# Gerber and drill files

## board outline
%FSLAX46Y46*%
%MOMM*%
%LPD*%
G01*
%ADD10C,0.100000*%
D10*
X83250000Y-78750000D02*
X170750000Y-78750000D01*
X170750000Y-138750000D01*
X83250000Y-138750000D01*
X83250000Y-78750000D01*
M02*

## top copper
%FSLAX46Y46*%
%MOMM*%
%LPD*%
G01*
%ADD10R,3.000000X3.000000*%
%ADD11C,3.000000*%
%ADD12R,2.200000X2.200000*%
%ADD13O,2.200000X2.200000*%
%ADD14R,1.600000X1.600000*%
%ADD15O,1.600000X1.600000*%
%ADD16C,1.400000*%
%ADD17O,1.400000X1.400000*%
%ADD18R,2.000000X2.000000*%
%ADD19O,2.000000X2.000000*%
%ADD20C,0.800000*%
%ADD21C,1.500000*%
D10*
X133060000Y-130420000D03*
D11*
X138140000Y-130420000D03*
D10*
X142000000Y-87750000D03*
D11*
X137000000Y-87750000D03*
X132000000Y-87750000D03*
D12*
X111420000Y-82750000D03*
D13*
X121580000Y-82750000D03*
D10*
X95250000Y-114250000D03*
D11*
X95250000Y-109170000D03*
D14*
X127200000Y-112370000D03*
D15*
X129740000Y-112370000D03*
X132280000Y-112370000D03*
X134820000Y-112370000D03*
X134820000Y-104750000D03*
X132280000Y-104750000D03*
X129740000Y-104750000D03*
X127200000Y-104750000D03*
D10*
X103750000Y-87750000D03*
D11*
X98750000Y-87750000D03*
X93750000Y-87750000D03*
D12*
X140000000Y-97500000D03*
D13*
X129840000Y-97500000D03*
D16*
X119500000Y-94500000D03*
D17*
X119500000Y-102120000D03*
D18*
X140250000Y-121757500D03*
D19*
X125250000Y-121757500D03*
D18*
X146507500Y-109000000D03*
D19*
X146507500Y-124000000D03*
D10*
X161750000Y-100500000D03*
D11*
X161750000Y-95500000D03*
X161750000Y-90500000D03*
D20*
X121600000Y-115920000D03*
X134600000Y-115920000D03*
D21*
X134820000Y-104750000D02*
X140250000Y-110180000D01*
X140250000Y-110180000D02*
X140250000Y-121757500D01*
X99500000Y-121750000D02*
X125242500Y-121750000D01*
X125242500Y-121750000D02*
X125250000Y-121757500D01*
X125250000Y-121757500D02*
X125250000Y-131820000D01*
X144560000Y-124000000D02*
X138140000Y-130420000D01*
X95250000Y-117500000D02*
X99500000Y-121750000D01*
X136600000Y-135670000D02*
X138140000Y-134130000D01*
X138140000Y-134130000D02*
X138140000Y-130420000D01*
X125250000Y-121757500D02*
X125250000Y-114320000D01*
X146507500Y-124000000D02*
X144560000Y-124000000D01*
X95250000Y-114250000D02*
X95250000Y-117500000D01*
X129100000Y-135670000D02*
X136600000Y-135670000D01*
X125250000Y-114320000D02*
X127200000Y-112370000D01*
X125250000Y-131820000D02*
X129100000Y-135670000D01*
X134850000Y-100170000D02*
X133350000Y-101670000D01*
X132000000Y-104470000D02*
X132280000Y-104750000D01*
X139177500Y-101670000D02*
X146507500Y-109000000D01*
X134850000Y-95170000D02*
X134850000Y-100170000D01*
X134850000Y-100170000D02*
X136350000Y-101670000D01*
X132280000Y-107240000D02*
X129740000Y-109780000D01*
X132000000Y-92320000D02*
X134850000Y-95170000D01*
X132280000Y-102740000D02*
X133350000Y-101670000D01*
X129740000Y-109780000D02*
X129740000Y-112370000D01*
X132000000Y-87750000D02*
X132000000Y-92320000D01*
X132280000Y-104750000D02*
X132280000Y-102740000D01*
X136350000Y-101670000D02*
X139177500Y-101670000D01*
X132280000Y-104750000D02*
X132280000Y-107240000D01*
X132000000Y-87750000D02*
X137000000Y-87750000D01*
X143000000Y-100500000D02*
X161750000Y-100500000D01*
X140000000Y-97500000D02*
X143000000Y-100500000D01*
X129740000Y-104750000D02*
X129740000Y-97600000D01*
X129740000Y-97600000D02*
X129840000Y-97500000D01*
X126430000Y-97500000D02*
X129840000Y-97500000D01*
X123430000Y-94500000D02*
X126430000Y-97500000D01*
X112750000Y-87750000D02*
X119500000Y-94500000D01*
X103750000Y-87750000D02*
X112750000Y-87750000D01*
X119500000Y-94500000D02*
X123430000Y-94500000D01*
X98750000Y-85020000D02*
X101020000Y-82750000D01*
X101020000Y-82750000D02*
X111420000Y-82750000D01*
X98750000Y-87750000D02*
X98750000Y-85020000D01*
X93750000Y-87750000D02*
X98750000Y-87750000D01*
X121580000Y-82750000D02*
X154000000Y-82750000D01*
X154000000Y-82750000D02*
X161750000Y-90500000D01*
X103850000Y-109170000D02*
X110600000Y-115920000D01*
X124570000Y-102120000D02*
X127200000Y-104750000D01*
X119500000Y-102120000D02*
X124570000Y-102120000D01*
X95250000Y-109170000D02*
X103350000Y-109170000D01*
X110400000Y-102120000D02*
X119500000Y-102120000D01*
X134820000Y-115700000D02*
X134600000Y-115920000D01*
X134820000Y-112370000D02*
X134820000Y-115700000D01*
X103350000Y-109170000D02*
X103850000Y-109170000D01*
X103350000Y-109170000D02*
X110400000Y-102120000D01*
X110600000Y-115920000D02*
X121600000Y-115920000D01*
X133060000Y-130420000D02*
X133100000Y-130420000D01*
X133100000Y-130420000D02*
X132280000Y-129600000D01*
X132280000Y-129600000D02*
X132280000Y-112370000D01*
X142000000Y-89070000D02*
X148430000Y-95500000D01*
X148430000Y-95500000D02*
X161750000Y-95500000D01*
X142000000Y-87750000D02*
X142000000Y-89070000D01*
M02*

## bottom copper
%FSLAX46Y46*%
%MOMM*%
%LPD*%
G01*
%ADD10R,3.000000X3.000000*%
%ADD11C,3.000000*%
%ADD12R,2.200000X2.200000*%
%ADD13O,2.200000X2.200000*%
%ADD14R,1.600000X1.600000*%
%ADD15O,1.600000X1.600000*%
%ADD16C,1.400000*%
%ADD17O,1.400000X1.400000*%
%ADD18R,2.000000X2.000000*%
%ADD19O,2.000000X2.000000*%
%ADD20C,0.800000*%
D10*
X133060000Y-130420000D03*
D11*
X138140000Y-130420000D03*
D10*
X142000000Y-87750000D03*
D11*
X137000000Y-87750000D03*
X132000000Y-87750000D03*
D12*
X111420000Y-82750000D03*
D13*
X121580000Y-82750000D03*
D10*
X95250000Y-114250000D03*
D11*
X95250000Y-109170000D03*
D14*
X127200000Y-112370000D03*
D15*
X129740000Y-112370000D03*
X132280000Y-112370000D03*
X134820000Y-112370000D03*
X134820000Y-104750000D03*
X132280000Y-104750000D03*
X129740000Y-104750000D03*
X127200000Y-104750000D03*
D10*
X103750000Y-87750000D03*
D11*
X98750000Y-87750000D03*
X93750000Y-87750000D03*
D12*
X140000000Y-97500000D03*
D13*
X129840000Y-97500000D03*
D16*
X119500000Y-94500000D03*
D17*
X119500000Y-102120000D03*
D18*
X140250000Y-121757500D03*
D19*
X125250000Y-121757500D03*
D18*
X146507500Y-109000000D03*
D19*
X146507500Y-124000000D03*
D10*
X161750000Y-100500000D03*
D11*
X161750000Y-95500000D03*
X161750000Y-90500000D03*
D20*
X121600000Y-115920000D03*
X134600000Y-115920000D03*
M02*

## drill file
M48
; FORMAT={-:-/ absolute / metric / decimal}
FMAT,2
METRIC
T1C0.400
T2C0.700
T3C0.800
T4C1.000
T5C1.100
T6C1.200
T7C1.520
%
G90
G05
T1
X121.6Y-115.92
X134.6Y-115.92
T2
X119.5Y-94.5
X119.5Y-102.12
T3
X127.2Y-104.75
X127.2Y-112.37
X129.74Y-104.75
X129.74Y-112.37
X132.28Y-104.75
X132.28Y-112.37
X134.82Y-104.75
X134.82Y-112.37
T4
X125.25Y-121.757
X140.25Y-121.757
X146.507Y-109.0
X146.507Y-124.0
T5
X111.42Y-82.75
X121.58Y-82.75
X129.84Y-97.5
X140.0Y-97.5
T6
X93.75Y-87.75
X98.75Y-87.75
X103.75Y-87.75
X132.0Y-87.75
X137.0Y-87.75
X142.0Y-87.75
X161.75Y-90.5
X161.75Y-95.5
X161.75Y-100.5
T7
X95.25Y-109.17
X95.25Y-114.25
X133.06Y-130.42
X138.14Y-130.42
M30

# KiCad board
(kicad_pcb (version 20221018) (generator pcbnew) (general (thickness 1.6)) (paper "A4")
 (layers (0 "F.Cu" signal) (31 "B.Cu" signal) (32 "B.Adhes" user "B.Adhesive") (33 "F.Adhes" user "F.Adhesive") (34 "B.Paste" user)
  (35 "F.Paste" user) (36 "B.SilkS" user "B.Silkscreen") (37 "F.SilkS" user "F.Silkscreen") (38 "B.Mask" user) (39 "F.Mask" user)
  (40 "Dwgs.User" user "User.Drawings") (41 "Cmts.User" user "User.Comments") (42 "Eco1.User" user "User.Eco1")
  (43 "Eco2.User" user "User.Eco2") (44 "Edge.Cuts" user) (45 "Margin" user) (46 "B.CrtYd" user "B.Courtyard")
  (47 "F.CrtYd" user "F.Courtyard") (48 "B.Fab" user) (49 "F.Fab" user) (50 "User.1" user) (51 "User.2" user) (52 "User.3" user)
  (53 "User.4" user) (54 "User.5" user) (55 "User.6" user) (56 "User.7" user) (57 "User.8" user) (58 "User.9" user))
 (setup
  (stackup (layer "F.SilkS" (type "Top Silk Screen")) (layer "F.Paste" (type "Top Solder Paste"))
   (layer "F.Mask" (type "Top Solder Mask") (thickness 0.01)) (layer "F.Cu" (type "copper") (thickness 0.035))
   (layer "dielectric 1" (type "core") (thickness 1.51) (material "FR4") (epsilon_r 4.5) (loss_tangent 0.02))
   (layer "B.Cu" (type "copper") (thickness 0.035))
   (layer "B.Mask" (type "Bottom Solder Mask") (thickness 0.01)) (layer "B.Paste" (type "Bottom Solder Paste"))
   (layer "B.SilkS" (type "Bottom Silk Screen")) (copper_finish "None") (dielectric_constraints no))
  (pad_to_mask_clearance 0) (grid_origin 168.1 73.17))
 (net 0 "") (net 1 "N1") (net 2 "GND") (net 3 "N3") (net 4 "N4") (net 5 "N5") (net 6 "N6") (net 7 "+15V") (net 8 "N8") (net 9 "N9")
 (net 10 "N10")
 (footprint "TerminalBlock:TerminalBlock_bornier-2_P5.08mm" (layer "F.Cu") (at 133.06 130.42)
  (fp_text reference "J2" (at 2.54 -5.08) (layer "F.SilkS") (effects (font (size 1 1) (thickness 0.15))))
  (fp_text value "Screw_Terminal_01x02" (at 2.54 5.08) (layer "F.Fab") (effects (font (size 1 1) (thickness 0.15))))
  (pad "1" thru_hole rect (at 0 0) (size 3 3) (drill 1.52) (layers "*.Cu" "*.Mask") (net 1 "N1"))
  (pad "2" thru_hole circle (at 5.08 0) (size 3 3) (drill 1.52) (layers "*.Cu" "*.Mask") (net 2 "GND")))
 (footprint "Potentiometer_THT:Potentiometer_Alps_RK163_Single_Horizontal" (layer "F.Cu") (at 142 87.75 -90)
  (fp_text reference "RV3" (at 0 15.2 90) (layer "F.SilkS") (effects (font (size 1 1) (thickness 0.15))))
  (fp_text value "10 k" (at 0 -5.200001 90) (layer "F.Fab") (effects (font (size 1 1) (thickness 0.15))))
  (pad "1" thru_hole rect (at 0 0 90) (size 3 3) (drill 1.2) (layers "*.Cu" "*.Mask") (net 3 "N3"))
  (pad "2" thru_hole circle (at 0 5 90) (size 3 3) (drill 1.2) (layers "*.Cu" "*.Mask") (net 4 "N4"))
  (pad "3" thru_hole circle (at 0 10 90) (size 3 3) (drill 1.2) (layers "*.Cu" "*.Mask") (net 4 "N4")))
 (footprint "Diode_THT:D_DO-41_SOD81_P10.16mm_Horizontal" (layer "F.Cu") (at 111.42 82.75)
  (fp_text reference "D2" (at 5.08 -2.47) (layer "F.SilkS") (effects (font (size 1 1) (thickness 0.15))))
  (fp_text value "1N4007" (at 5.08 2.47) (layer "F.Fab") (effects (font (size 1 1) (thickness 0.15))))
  (pad "1" thru_hole rect (at 0 0) (size 2.2 2.2) (drill 1.1) (layers "*.Cu" "*.Mask") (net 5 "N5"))
  (pad "2" thru_hole oval (at 10.16 0) (size 2.2 2.2) (drill 1.1) (layers "*.Cu" "*.Mask") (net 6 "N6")))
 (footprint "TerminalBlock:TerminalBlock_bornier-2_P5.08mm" (layer "F.Cu") (at 95.25 114.25 90)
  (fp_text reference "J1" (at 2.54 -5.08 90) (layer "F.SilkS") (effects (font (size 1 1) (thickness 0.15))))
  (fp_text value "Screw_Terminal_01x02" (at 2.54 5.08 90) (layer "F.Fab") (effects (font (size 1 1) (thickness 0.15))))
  (pad "1" thru_hole rect (at 0 0 90) (size 3 3) (drill 1.52) (layers "*.Cu" "*.Mask") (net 2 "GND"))
  (pad "2" thru_hole circle (at 5.08 0 90) (size 3 3) (drill 1.52) (layers "*.Cu" "*.Mask") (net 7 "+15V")))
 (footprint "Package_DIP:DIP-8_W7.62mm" (layer "F.Cu") (at 127.2 112.37 90)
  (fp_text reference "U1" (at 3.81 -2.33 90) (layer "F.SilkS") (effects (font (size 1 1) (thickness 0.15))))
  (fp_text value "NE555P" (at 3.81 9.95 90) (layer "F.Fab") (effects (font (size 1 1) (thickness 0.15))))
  (pad "1" thru_hole rect (at 0 0 90) (size 1.6 1.6) (drill 0.8) (layers "*.Cu" "*.Mask") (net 2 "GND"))
  (pad "2" thru_hole oval (at 0 2.54 90) (size 1.6 1.6) (drill 0.8) (layers "*.Cu" "*.Mask") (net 4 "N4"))
  (pad "3" thru_hole oval (at 0 5.08 90) (size 1.6 1.6) (drill 0.8) (layers "*.Cu" "*.Mask") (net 1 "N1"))
  (pad "4" thru_hole oval (at 0 7.62 90) (size 1.6 1.6) (drill 0.8) (layers "*.Cu" "*.Mask") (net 7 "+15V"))
  (pad "5" thru_hole oval (at 7.62 7.62 90) (size 1.6 1.6) (drill 0.8) (layers "*.Cu" "*.Mask") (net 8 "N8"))
  (pad "6" thru_hole oval (at 7.62 5.08 90) (size 1.6 1.6) (drill 0.8) (layers "*.Cu" "*.Mask") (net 4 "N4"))
  (pad "7" thru_hole oval (at 7.62 2.54 90) (size 1.6 1.6) (drill 0.8) (layers "*.Cu" "*.Mask") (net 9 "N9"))
  (pad "8" thru_hole oval (at 7.62 0 90) (size 1.6 1.6) (drill 0.8) (layers "*.Cu" "*.Mask") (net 7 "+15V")))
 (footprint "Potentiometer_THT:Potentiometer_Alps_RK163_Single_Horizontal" (layer "F.Cu") (at 103.75 87.75 -90)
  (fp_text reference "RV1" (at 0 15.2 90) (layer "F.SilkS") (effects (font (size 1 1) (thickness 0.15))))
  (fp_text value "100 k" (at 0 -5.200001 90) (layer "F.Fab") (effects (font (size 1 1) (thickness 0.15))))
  (pad "1" thru_hole rect (at 0 0 90) (size 3 3) (drill 1.2) (layers "*.Cu" "*.Mask") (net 9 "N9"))
  (pad "2" thru_hole circle (at 0 5 90) (size 3 3) (drill 1.2) (layers "*.Cu" "*.Mask") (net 5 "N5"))
  (pad "3" thru_hole circle (at 0 10 90) (size 3 3) (drill 1.2) (layers "*.Cu" "*.Mask") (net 5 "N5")))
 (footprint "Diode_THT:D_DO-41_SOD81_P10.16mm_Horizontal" (layer "F.Cu") (at 140 97.5 180)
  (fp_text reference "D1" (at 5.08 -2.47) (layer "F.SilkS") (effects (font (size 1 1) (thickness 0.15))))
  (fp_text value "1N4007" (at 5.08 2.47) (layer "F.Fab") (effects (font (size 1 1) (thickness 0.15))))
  (pad "1" thru_hole rect (at 0 0 180) (size 2.2 2.2) (drill 1.1) (layers "*.Cu" "*.Mask") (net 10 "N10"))
  (pad "2" thru_hole oval (at 10.16 0 180) (size 2.2 2.2) (drill 1.1) (layers "*.Cu" "*.Mask") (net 9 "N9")))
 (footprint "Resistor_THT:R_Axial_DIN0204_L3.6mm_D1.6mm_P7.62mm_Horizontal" (layer "F.Cu") (at 119.5 94.5 -90)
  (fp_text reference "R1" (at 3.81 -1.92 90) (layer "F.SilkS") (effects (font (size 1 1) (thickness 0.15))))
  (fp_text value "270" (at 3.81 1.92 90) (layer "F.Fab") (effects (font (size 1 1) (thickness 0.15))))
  (pad "1" thru_hole circle (at 0 0 270) (size 1.4 1.4) (drill 0.7) (layers "*.Cu" "*.Mask") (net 9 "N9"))
  (pad "2" thru_hole oval (at 7.62 0 270) (size 1.4 1.4) (drill 0.7) (layers "*.Cu" "*.Mask") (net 7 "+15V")))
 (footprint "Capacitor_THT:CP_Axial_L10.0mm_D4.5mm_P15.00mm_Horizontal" (layer "F.Cu") (at 140.25 121.7575 180)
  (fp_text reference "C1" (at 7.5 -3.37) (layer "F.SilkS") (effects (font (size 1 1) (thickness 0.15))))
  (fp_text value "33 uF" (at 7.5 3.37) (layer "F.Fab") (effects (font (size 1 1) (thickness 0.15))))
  (pad "1" thru_hole rect (at 0 0 180) (size 2 2) (drill 1) (layers "*.Cu" "*.Mask") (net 8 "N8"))
  (pad "2" thru_hole oval (at 15 0 180) (size 2 2) (drill 1) (layers "*.Cu" "*.Mask") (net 2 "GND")))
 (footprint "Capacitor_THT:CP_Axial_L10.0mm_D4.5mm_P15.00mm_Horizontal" (layer "F.Cu") (at 146.5075 109 -90)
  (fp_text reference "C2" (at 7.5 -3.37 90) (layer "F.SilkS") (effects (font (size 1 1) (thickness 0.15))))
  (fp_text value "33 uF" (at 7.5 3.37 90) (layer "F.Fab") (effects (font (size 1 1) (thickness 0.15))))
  (pad "1" thru_hole rect (at 0 0 270) (size 2 2) (drill 1) (layers "*.Cu" "*.Mask") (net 4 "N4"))
  (pad "2" thru_hole oval (at 15 0 270) (size 2 2) (drill 1) (layers "*.Cu" "*.Mask") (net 2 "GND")))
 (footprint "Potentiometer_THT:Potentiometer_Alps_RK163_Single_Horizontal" (layer "F.Cu") (at 161.75 100.5 180)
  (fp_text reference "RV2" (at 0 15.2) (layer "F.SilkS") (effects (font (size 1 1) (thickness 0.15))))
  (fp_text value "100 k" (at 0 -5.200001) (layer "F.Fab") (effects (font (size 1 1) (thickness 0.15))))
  (pad "1" thru_hole rect (at 0 0) (size 3 3) (drill 1.2) (layers "*.Cu" "*.Mask") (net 10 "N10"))
  (pad "2" thru_hole circle (at 0 5) (size 3 3) (drill 1.2) (layers "*.Cu" "*.Mask") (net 3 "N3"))
  (pad "3" thru_hole circle (at 0 10) (size 3 3) (drill 1.2) (layers "*.Cu" "*.Mask") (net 6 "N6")))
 (gr_rect (start 83.25 78.75) (end 170.75 138.75) (stroke (width 0.1) (type default)) (fill none) (layer "Edge.Cuts"))
 (segment (start 134.82 104.75) (end 140.25 110.18) (width 1.5) (layer "F.Cu") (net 8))
 (segment (start 140.25 110.18) (end 140.25 121.7575) (width 1.5) (layer "F.Cu") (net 8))
 (segment (start 99.5 121.75) (end 125.2425 121.75) (width 1.5) (layer "F.Cu") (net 2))
 (segment (start 125.2425 121.75) (end 125.25 121.7575) (width 1.5) (layer "F.Cu") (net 2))
 (segment (start 125.25 121.7575) (end 125.25 131.82) (width 1.5) (layer "F.Cu") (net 2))
 (segment (start 144.56 124) (end 138.14 130.42) (width 1.5) (layer "F.Cu") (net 2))
 (segment (start 95.25 117.5) (end 99.5 121.75) (width 1.5) (layer "F.Cu") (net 2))
 (segment (start 136.6 135.67) (end 138.14 134.13) (width 1.5) (layer "F.Cu") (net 2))
 (segment (start 138.14 134.13) (end 138.14 130.42) (width 1.5) (layer "F.Cu") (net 2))
 (segment (start 125.25 121.7575) (end 125.25 114.32) (width 1.5) (layer "F.Cu") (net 2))
 (segment (start 146.5075 124) (end 144.56 124) (width 1.5) (layer "F.Cu") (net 2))
 (segment (start 95.25 114.25) (end 95.25 117.5) (width 1.5) (layer "F.Cu") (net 2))
 (segment (start 129.1 135.67) (end 136.6 135.67) (width 1.5) (layer "F.Cu") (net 2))
 (segment (start 125.25 114.32) (end 127.2 112.37) (width 1.5) (layer "F.Cu") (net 2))
 (segment (start 125.25 131.82) (end 129.1 135.67) (width 1.5) (layer "F.Cu") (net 2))
 (segment (start 134.85 100.17) (end 133.35 101.67) (width 1.5) (layer "F.Cu") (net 4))
 (segment (start 132 104.47) (end 132.28 104.75) (width 1.5) (layer "F.Cu") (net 4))
 (segment (start 139.1775 101.67) (end 146.5075 109) (width 1.5) (layer "F.Cu") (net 4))
 (segment (start 134.85 95.17) (end 134.85 100.17) (width 1.5) (layer "F.Cu") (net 4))
 (segment (start 134.85 100.17) (end 136.35 101.67) (width 1.5) (layer "F.Cu") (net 4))
 (segment (start 132.28 107.24) (end 129.74 109.78) (width 1.5) (layer "F.Cu") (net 4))
 (segment (start 132 92.32) (end 134.85 95.17) (width 1.5) (layer "F.Cu") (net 4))
 (segment (start 132.28 102.74) (end 133.35 101.67) (width 1.5) (layer "F.Cu") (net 4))
 (segment (start 129.74 109.78) (end 129.74 112.37) (width 1.5) (layer "F.Cu") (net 4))
 (segment (start 132 87.75) (end 132 92.32) (width 1.5) (layer "F.Cu") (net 4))
 (segment (start 132.28 104.75) (end 132.28 102.74) (width 1.5) (layer "F.Cu") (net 4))
 (segment (start 136.35 101.67) (end 139.1775 101.67) (width 1.5) (layer "F.Cu") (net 4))
 (segment (start 132.28 104.75) (end 132.28 107.24) (width 1.5) (layer "F.Cu") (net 4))
 (segment (start 132 87.75) (end 137 87.75) (width 1.5) (layer "F.Cu") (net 4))
 (segment (start 143 100.5) (end 161.75 100.5) (width 1.5) (layer "F.Cu") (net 10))
 (segment (start 140 97.5) (end 143 100.5) (width 1.5) (layer "F.Cu") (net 10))
 (segment (start 129.74 104.75) (end 129.74 97.6) (width 1.5) (layer "F.Cu") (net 9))
 (segment (start 129.74 97.6) (end 129.84 97.5) (width 1.5) (layer "F.Cu") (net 9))
 (segment (start 126.43 97.5) (end 129.84 97.5) (width 1.5) (layer "F.Cu") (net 9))
 (segment (start 123.43 94.5) (end 126.43 97.5) (width 1.5) (layer "F.Cu") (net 9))
 (segment (start 112.75 87.75) (end 119.5 94.5) (width 1.5) (layer "F.Cu") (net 9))
 (segment (start 103.75 87.75) (end 112.75 87.75) (width 1.5) (layer "F.Cu") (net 9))
 (segment (start 119.5 94.5) (end 123.43 94.5) (width 1.5) (layer "F.Cu") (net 9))
 (segment (start 98.75 85.02) (end 101.02 82.75) (width 1.5) (layer "F.Cu") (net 5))
 (segment (start 101.02 82.75) (end 111.42 82.75) (width 1.5) (layer "F.Cu") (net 5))
 (segment (start 98.75 87.75) (end 98.75 85.02) (width 1.5) (layer "F.Cu") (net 5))
 (segment (start 93.75 87.75) (end 98.75 87.75) (width 1.5) (layer "F.Cu") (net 5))
 (segment (start 121.58 82.75) (end 154 82.75) (width 1.5) (layer "F.Cu") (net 6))
 (segment (start 154 82.75) (end 161.75 90.5) (width 1.5) (layer "F.Cu") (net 6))
 (segment (start 103.85 109.17) (end 110.6 115.92) (width 1.5) (layer "F.Cu") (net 7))
 (segment (start 124.57 102.12) (end 127.2 104.75) (width 1.5) (layer "F.Cu") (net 7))
 (segment (start 119.5 102.12) (end 124.57 102.12) (width 1.5) (layer "F.Cu") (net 7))
 (segment (start 95.25 109.17) (end 103.35 109.17) (width 1.5) (layer "F.Cu") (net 7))
 (segment (start 110.4 102.12) (end 119.5 102.12) (width 1.5) (layer "F.Cu") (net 7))
 (segment (start 134.82 115.7) (end 134.6 115.92) (width 1.5) (layer "F.Cu") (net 7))
 (segment (start 134.82 112.37) (end 134.82 115.7) (width 1.5) (layer "F.Cu") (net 7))
 (segment (start 103.35 109.17) (end 103.85 109.17) (width 1.5) (layer "F.Cu") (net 7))
 (segment (start 103.35 109.17) (end 110.4 102.12) (width 1.5) (layer "F.Cu") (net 7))
 (segment (start 110.6 115.92) (end 121.6 115.92) (width 1.5) (layer "F.Cu") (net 7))
 (via (at 121.6 115.92) (size 0.8) (drill 0.4) (layers "F.Cu" "B.Cu") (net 7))
 (via (at 134.6 115.92) (size 0.8) (drill 0.4) (layers "F.Cu" "B.Cu") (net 7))
 (segment (start 133.06 130.42) (end 133.1 130.42) (width 1.5) (layer "F.Cu") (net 1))
 (segment (start 133.1 130.42) (end 132.28 129.6) (width 1.5) (layer "F.Cu") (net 1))
 (segment (start 132.28 129.6) (end 132.28 112.37) (width 1.5) (layer "F.Cu") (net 1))
 (segment (start 142 89.07) (end 148.43 95.5) (width 1.5) (layer "F.Cu") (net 3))
 (segment (start 148.43 95.5) (end 161.75 95.5) (width 1.5) (layer "F.Cu") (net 3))
 (segment (start 142 87.75) (end 142 89.07) (width 1.5) (layer "F.Cu") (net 3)))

